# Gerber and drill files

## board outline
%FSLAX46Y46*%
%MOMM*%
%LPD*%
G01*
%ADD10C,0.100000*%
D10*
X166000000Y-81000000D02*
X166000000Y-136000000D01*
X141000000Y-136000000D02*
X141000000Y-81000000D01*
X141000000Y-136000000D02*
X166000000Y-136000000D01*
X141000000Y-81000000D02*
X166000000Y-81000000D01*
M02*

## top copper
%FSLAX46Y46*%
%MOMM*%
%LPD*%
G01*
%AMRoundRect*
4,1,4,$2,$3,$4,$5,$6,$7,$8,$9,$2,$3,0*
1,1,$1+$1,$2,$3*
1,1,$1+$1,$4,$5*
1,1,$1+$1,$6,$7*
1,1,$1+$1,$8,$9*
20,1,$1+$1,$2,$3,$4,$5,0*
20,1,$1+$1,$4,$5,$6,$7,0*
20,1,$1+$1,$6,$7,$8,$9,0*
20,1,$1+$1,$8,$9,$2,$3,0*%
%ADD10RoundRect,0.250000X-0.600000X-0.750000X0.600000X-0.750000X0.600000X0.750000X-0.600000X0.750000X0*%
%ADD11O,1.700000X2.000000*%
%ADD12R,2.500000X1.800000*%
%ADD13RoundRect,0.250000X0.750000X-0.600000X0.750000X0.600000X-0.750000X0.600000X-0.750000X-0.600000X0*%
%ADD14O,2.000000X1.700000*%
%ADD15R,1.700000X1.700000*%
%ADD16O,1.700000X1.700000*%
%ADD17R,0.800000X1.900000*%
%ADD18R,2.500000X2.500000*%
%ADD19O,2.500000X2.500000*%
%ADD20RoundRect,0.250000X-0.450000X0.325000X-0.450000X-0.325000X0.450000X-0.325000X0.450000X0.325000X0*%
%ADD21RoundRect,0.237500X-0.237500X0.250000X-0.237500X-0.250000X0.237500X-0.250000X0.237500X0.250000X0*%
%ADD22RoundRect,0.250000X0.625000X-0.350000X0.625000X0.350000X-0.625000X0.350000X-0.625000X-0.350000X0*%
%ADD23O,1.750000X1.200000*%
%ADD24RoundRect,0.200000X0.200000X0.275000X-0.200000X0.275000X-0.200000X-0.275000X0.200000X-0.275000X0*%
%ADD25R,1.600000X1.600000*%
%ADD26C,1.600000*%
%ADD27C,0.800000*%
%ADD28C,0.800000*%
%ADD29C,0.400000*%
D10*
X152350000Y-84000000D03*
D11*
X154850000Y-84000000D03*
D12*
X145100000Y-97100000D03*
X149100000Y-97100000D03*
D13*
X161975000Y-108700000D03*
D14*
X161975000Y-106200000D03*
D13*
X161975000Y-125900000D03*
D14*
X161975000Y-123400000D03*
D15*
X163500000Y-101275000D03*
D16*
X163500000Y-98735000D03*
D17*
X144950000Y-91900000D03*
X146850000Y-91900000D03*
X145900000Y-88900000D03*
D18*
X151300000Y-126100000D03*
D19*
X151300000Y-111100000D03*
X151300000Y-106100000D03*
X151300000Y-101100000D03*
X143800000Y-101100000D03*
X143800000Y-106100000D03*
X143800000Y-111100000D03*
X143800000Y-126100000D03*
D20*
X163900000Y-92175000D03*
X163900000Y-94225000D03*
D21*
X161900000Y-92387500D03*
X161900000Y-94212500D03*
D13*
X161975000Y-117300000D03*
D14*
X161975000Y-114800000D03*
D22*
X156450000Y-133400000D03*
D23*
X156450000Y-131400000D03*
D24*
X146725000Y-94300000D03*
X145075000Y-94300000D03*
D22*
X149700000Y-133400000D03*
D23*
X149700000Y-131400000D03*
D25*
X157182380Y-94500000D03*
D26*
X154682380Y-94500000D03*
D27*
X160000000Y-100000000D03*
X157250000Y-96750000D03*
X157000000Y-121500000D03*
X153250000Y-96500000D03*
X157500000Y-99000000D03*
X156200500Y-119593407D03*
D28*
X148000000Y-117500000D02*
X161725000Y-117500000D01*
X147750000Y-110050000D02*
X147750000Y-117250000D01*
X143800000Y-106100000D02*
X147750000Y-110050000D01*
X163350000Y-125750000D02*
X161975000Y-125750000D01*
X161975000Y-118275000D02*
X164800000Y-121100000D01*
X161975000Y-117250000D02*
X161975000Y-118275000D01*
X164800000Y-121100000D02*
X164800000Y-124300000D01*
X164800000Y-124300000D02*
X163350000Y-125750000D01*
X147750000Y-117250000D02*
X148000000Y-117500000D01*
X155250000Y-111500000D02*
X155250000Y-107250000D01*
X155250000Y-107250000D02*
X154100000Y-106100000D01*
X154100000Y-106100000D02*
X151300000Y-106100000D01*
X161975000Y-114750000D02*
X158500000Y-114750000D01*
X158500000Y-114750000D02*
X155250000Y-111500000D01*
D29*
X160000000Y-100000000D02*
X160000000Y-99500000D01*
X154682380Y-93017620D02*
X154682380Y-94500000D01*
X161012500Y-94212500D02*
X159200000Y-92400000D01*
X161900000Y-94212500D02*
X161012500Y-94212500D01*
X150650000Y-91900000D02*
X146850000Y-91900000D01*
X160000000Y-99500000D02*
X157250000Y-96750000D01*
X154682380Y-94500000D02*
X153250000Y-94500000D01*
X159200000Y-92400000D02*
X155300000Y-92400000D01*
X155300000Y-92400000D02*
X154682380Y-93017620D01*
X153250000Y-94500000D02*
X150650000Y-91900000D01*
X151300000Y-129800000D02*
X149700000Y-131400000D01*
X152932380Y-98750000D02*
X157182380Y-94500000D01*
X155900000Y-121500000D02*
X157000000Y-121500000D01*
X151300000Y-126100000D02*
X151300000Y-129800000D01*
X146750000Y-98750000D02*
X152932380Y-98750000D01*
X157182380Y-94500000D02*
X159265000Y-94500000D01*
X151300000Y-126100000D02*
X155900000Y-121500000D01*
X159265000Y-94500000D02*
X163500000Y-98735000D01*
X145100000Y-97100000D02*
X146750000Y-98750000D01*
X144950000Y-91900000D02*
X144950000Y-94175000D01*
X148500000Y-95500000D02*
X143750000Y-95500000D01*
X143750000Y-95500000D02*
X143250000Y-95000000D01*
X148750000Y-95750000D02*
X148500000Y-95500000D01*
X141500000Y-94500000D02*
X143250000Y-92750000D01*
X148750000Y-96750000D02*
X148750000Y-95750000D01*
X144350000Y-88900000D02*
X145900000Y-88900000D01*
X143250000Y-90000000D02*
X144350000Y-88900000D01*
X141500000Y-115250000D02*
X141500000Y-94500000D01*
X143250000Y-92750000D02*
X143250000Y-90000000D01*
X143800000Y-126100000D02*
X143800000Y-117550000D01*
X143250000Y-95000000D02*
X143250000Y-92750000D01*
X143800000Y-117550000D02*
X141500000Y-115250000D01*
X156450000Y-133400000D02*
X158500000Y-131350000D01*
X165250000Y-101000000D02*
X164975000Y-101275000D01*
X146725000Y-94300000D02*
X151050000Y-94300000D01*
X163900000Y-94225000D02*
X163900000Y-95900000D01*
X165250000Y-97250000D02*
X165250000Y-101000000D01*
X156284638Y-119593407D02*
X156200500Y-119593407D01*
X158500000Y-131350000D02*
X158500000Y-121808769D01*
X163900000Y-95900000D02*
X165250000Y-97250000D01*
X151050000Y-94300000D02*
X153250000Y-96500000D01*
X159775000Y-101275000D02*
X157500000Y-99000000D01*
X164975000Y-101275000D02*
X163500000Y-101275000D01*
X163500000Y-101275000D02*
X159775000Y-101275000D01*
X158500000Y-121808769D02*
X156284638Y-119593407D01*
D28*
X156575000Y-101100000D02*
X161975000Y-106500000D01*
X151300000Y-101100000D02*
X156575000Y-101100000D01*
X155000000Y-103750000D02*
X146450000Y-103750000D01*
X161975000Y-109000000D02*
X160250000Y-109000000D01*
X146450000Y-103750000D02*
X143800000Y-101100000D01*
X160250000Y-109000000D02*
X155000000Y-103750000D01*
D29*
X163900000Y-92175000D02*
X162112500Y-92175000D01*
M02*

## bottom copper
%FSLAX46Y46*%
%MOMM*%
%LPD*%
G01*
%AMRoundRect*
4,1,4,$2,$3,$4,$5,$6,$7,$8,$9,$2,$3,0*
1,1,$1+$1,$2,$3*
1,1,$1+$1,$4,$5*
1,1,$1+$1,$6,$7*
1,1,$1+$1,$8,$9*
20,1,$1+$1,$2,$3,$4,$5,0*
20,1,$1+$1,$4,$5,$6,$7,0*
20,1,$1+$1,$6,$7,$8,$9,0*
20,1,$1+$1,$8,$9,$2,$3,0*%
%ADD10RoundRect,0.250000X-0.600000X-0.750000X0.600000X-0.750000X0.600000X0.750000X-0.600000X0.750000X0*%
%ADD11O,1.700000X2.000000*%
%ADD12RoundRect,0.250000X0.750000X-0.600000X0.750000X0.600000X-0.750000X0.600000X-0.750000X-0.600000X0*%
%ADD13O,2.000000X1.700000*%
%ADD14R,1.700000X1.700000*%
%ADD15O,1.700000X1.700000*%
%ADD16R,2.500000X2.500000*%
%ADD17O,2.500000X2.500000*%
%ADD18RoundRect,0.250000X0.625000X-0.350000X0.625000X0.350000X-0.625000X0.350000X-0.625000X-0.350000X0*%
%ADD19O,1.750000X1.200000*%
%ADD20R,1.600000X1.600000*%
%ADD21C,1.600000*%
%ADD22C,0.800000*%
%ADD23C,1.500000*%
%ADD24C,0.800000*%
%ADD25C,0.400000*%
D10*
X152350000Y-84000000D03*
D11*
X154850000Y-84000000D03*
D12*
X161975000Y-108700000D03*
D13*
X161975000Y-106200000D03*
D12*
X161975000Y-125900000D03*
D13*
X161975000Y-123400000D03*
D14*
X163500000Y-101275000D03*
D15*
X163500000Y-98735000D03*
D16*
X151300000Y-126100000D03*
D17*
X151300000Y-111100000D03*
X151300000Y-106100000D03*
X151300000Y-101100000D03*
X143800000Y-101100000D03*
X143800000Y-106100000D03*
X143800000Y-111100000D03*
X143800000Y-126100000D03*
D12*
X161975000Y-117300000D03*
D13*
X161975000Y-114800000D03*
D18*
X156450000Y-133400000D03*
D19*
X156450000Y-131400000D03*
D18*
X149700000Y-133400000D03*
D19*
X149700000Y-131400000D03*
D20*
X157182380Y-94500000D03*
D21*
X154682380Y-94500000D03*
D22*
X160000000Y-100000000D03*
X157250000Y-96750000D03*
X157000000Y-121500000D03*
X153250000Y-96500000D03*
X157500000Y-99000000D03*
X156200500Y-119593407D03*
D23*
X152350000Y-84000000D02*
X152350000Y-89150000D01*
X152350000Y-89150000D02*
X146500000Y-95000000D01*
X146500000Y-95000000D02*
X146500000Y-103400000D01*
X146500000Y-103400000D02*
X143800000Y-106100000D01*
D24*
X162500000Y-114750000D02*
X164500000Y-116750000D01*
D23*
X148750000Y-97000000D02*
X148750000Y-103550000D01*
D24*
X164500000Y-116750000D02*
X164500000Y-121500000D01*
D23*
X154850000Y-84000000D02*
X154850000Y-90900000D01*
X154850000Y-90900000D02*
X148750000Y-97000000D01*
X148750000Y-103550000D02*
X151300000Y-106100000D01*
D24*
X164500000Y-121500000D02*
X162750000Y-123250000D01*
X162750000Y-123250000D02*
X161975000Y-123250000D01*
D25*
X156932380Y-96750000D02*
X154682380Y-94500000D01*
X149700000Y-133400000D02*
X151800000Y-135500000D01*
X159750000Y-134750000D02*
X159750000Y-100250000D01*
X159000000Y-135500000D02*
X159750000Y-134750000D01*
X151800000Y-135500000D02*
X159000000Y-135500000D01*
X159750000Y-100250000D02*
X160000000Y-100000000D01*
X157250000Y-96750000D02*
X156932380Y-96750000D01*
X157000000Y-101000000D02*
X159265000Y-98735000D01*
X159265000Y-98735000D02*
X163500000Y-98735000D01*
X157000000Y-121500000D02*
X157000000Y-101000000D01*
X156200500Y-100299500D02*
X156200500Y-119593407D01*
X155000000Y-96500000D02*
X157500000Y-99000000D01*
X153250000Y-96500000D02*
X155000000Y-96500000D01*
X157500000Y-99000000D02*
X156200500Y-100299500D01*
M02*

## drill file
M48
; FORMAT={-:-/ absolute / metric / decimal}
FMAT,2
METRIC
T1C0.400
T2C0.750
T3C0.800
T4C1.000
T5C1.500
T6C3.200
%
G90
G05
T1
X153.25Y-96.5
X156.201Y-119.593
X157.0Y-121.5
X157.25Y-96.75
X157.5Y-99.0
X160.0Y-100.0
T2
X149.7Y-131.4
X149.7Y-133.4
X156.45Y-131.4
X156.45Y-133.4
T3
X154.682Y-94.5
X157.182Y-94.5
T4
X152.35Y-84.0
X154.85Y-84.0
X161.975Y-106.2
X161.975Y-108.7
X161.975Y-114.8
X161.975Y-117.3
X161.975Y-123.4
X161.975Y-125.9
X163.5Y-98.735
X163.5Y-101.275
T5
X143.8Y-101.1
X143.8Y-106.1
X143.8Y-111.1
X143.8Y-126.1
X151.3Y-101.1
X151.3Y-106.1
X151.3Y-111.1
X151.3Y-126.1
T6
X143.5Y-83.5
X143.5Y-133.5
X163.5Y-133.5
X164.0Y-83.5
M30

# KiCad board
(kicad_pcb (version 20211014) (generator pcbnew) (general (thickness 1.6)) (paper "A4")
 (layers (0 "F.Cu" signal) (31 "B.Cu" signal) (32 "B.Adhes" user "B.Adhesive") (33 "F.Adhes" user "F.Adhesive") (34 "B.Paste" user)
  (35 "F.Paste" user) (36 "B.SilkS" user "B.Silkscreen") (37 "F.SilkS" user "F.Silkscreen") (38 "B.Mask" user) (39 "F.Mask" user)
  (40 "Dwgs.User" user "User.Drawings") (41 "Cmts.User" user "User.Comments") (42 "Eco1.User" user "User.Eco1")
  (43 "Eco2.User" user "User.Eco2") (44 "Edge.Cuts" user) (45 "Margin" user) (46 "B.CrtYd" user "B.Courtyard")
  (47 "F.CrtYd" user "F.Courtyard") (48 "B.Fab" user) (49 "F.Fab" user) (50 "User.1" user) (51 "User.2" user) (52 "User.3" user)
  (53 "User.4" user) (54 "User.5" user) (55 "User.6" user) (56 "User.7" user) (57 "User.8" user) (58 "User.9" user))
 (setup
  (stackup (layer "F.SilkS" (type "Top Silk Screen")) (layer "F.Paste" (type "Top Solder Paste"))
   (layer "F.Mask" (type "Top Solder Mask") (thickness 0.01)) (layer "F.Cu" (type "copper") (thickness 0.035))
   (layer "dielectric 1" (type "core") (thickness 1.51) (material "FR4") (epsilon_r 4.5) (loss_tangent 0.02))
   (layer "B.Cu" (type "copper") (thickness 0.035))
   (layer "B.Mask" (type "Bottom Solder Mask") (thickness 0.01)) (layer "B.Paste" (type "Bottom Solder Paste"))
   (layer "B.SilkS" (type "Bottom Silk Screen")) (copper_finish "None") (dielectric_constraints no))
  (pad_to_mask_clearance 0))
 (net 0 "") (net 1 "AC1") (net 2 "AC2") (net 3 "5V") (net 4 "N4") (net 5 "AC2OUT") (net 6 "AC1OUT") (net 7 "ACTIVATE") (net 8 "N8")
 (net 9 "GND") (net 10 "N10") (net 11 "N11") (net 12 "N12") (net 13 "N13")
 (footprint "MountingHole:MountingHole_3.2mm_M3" (layer "F.Cu") (at 163.5 133.5)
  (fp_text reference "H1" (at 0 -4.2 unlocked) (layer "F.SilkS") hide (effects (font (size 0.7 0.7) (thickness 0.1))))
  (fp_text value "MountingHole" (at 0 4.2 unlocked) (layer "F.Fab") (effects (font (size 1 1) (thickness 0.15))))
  (pad "" np_thru_hole circle (at 0 0) (size 3.2 3.2) (drill 3.2) (layers *.Cu *.Mask)))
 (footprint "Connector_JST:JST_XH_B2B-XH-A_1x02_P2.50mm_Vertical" (layer "F.Cu") (at 152.35 84)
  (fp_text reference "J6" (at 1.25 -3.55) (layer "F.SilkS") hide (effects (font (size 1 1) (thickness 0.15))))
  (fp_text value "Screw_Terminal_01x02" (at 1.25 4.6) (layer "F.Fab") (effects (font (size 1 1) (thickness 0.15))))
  (pad "1" thru_hole roundrect (at 0 0) (size 1.7 2) (drill 1) (layers *.Cu *.Mask) (roundrect_rratio 0.1470588235) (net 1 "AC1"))
  (pad "2" thru_hole oval (at 2.5 0) (size 1.7 2) (drill 1) (layers *.Cu *.Mask) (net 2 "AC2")))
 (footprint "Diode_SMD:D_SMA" (layer "F.Cu") (at 147.1 97.1)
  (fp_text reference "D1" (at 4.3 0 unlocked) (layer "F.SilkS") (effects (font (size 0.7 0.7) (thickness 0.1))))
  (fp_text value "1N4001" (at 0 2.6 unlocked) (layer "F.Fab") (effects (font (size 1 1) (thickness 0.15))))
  (pad "1" smd rect (at -2 0) (size 2.5 1.8) (layers "F.Cu" "F.Paste" "F.Mask") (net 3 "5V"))
  (pad "2" smd rect (at 2 0) (size 2.5 1.8) (layers "F.Cu" "F.Paste" "F.Mask") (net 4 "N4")))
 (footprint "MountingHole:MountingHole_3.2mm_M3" (layer "F.Cu") (at 164 83.5)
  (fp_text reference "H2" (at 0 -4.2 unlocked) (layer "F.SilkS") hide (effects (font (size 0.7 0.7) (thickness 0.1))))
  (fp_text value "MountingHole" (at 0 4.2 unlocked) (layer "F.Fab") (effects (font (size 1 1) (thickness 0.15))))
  (pad "" np_thru_hole circle (at 0 0) (size 3.2 3.2) (drill 3.2) (layers *.Cu *.Mask)))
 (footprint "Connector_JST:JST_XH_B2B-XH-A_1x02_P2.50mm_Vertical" (layer "F.Cu") (at 161.975 108.7 90)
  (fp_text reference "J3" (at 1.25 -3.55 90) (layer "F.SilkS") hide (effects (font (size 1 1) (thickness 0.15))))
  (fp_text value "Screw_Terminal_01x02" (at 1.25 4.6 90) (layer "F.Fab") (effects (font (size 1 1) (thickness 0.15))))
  (pad "1" thru_hole roundrect (at 0 0 90) (size 1.7 2) (drill 1) (layers *.Cu *.Mask) (roundrect_rratio 0.1470588235) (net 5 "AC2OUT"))
  (pad "2" thru_hole oval (at 2.5 0 90) (size 1.7 2) (drill 1) (layers *.Cu *.Mask) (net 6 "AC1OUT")))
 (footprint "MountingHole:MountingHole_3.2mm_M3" (layer "F.Cu") (at 143.5 83.5)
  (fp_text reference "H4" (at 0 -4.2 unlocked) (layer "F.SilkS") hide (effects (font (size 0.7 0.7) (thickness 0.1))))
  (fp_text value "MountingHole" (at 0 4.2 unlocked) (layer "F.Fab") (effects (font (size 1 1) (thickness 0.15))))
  (pad "" np_thru_hole circle (at 0 0) (size 3.2 3.2) (drill 3.2) (layers *.Cu *.Mask)))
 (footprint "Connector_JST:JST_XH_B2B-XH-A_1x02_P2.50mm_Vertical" (layer "F.Cu") (at 161.975 125.9 90)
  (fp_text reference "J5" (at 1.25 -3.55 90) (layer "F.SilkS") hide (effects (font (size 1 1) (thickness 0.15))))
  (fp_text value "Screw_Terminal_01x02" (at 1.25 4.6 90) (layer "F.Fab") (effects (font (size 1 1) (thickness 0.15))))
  (pad "1" thru_hole roundrect (at 0 0 90) (size 1.7 2) (drill 1) (layers *.Cu *.Mask) (roundrect_rratio 0.1470588235) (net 1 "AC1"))
  (pad "2" thru_hole oval (at 2.5 0 90) (size 1.7 2) (drill 1) (layers *.Cu *.Mask) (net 2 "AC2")))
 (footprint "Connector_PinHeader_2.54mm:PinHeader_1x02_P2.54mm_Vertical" (layer "F.Cu") (at 163.5 101.275 180)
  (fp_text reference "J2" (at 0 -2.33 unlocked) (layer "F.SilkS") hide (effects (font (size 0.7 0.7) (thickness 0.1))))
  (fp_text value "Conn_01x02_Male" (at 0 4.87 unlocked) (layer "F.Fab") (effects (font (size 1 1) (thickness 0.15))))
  (pad "1" thru_hole rect (at 0 0 180) (size 1.7 1.7) (drill 1) (layers *.Cu *.Mask) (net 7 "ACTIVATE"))
  (pad "2" thru_hole oval (at 0 2.54 180) (size 1.7 1.7) (drill 1) (layers *.Cu *.Mask) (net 3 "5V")))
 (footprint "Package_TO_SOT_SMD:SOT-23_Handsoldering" (layer "F.Cu") (at 145.9 90.4 90)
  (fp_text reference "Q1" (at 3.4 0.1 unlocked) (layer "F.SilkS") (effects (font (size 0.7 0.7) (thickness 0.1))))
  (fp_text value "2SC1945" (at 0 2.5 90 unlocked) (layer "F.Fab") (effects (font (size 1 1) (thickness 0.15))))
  (pad "1" smd rect (at -1.5 -0.95 90) (size 1.9 0.8) (layers "F.Cu" "F.Paste" "F.Mask") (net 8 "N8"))
  (pad "2" smd rect (at -1.5 0.95 90) (size 1.9 0.8) (layers "F.Cu" "F.Paste" "F.Mask") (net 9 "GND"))
  (pad "3" smd rect (at 1.5 0 90) (size 1.9 0.8) (layers "F.Cu" "F.Paste" "F.Mask") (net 4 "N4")))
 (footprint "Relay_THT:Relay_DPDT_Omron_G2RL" (layer "F.Cu") (at 151.3 126.1 90)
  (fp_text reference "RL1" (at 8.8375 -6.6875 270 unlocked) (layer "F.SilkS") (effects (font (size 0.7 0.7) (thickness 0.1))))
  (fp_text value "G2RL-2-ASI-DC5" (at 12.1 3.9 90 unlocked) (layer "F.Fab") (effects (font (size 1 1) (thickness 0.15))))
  (pad "1" thru_hole rect (at 0 0 180) (size 2.5 2.5) (drill 1.5) (layers *.Cu *.Mask) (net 3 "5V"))
  (pad "2" thru_hole oval (at 15 0 180) (size 2.5 2.5) (drill 1.5) (layers *.Cu *.Mask) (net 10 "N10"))
  (pad "3" thru_hole oval (at 20 0 180) (size 2.5 2.5) (drill 1.5) (layers *.Cu *.Mask) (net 2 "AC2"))
  (pad "4" thru_hole oval (at 25 0 180) (size 2.5 2.5) (drill 1.5) (layers *.Cu *.Mask) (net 6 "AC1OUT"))
  (pad "5" thru_hole oval (at 25 -7.5 180) (size 2.5 2.5) (drill 1.5) (layers *.Cu *.Mask) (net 5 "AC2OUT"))
  (pad "6" thru_hole oval (at 20 -7.5 180) (size 2.5 2.5) (drill 1.5) (layers *.Cu *.Mask) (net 1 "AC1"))
  (pad "7" thru_hole oval (at 15 -7.5 180) (size 2.5 2.5) (drill 1.5) (layers *.Cu *.Mask) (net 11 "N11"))
  (pad "8" thru_hole oval (at 0 -7.5 180) (size 2.5 2.5) (drill 1.5) (layers *.Cu *.Mask) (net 4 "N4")))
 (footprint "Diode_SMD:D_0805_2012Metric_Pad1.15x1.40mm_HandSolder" (layer "F.Cu") (at 163.9 93.2 -90)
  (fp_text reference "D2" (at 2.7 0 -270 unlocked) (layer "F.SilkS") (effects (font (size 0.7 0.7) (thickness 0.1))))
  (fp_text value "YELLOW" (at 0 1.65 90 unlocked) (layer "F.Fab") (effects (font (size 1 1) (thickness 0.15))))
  (pad "1" smd roundrect (at -1.025 0 270) (size 1.15 1.4) (layers "F.Cu" "F.Paste" "F.Mask") (roundrect_rratio 0.2173913043) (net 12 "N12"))
  (pad "2" smd roundrect (at 1.025 0 270) (size 1.15 1.4) (layers "F.Cu" "F.Paste" "F.Mask") (roundrect_rratio 0.2173913043)
   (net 7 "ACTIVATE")))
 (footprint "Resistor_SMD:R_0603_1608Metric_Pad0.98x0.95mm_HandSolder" (layer "F.Cu") (at 161.9 93.3 -90)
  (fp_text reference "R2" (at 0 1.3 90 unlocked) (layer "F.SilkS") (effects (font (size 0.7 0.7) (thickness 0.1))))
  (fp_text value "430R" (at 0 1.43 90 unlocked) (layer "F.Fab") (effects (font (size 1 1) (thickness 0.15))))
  (pad "1" smd roundrect (at -0.9125 0 270) (size 0.975 0.95) (layers "F.Cu" "F.Paste" "F.Mask") (roundrect_rratio 0.25) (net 12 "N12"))
  (pad "2" smd roundrect (at 0.9125 0 270) (size 0.975 0.95) (layers "F.Cu" "F.Paste" "F.Mask") (roundrect_rratio 0.25) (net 9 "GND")))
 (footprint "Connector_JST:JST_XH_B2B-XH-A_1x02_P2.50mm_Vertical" (layer "F.Cu") (at 161.975 117.3 90)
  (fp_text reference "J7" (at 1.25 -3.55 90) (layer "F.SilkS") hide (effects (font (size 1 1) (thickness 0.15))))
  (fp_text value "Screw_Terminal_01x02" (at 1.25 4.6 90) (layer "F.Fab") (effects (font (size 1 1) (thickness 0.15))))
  (pad "1" thru_hole roundrect (at 0 0 90) (size 1.7 2) (drill 1) (layers *.Cu *.Mask) (roundrect_rratio 0.1470588235) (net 1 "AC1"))
  (pad "2" thru_hole oval (at 2.5 0 90) (size 1.7 2) (drill 1) (layers *.Cu *.Mask) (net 2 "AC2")))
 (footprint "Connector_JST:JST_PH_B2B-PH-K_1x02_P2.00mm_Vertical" (layer "F.Cu") (at 156.45 133.4 90)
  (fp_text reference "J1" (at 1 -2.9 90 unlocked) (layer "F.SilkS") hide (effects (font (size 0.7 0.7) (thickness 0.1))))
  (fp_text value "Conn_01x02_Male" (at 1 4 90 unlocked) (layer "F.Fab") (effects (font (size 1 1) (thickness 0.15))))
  (pad "1" thru_hole roundrect (at 0 0 90) (size 1.2 1.75) (drill 0.75) (layers *.Cu *.Mask) (roundrect_rratio 0.2083333333)
   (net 7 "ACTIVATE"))
  (pad "2" thru_hole oval (at 2 0 90) (size 1.2 1.75) (drill 0.75) (layers *.Cu *.Mask) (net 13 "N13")))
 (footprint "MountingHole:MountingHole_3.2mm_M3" (layer "F.Cu") (at 143.5 133.5)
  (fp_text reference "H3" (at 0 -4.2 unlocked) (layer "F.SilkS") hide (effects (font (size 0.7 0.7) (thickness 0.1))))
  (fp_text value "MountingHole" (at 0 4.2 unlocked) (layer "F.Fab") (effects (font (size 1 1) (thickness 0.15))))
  (pad "" np_thru_hole circle (at 0 0) (size 3.2 3.2) (drill 3.2) (layers *.Cu *.Mask)))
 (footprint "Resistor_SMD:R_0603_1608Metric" (layer "F.Cu") (at 145.9 94.3 180)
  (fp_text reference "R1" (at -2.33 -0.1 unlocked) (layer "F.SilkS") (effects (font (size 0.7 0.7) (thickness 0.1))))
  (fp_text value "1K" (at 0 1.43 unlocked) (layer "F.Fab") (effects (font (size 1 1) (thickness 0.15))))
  (pad "1" smd roundrect (at -0.825 0 180) (size 0.8 0.95) (layers "F.Cu" "F.Paste" "F.Mask") (roundrect_rratio 0.25) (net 7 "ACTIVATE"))
  (pad "2" smd roundrect (at 0.825 0 180) (size 0.8 0.95) (layers "F.Cu" "F.Paste" "F.Mask") (roundrect_rratio 0.25) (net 8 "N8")))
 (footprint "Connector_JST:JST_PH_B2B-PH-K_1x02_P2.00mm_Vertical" (layer "F.Cu") (at 149.7 133.4 90)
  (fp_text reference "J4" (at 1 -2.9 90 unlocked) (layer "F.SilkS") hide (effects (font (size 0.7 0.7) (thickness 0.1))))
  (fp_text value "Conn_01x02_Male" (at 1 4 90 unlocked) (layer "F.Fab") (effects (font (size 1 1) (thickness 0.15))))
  (pad "1" thru_hole roundrect (at 0 0 90) (size 1.2 1.75) (drill 0.75) (layers *.Cu *.Mask) (roundrect_rratio 0.2083333333) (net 9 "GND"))
  (pad "2" thru_hole oval (at 2 0 90) (size 1.2 1.75) (drill 0.75) (layers *.Cu *.Mask) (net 3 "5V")))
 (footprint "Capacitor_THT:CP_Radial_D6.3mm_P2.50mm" (layer "F.Cu") (at 157.18238 94.5 180)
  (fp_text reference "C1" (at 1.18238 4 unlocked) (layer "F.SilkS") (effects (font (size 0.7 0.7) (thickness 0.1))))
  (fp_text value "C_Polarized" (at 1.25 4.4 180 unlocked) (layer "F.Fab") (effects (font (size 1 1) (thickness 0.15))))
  (pad "1" thru_hole rect (at 0 0 180) (size 1.6 1.6) (drill 0.8) (layers *.Cu *.Mask) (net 3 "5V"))
  (pad "2" thru_hole circle (at 2.5 0 180) (size 1.6 1.6) (drill 0.8) (layers *.Cu *.Mask) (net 9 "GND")))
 (gr_line (start 166 81) (end 166 136) (layer "Edge.Cuts") (width 0.1))
 (gr_line (start 141 136) (end 141 81) (layer "Edge.Cuts") (width 0.1))
 (gr_line (start 141 136) (end 166 136) (layer "Edge.Cuts") (width 0.1))
 (gr_line (start 141 81) (end 166 81) (layer "Edge.Cuts") (width 0.1))
 (segment (start 148 117.5) (end 161.725 117.5) (width 0.8) (layer "F.Cu") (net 1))
 (segment (start 147.75 110.05) (end 147.75 117.25) (width 0.8) (layer "F.Cu") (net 1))
 (segment (start 143.8 106.1) (end 147.75 110.05) (width 0.8) (layer "F.Cu") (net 1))
 (segment (start 163.35 125.75) (end 161.975 125.75) (width 0.8) (layer "F.Cu") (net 1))
 (segment (start 161.975 118.275) (end 164.8 121.1) (width 0.8) (layer "F.Cu") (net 1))
 (segment (start 161.975 117.25) (end 161.975 118.275) (width 0.8) (layer "F.Cu") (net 1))
 (segment (start 164.8 121.1) (end 164.8 124.3) (width 0.8) (layer "F.Cu") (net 1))
 (segment (start 164.8 124.3) (end 163.35 125.75) (width 0.8) (layer "F.Cu") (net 1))
 (segment (start 147.75 117.25) (end 148 117.5) (width 0.8) (layer "F.Cu") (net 1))
 (segment (start 152.35 84) (end 152.35 89.15) (width 1.5) (layer "B.Cu") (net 1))
 (segment (start 152.35 89.15) (end 146.5 95) (width 1.5) (layer "B.Cu") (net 1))
 (segment (start 146.5 95) (end 146.5 103.4) (width 1.5) (layer "B.Cu") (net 1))
 (segment (start 146.5 103.4) (end 143.8 106.1) (width 1.5) (layer "B.Cu") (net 1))
 (segment (start 155.25 111.5) (end 155.25 107.25) (width 0.8) (layer "F.Cu") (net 2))
 (segment (start 155.25 107.25) (end 154.1 106.1) (width 0.8) (layer "F.Cu") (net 2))
 (segment (start 154.1 106.1) (end 151.3 106.1) (width 0.8) (layer "F.Cu") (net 2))
 (segment (start 161.975 114.75) (end 158.5 114.75) (width 0.8) (layer "F.Cu") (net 2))
 (segment (start 158.5 114.75) (end 155.25 111.5) (width 0.8) (layer "F.Cu") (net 2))
 (segment (start 162.5 114.75) (end 164.5 116.75) (width 0.8) (layer "B.Cu") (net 2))
 (segment (start 148.75 97) (end 148.75 103.55) (width 1.5) (layer "B.Cu") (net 2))
 (segment (start 164.5 116.75) (end 164.5 121.5) (width 0.8) (layer "B.Cu") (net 2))
 (segment (start 154.85 84) (end 154.85 90.9) (width 1.5) (layer "B.Cu") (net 2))
 (segment (start 154.85 90.9) (end 148.75 97) (width 1.5) (layer "B.Cu") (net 2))
 (segment (start 148.75 103.55) (end 151.3 106.1) (width 1.5) (layer "B.Cu") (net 2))
 (segment (start 164.5 121.5) (end 162.75 123.25) (width 0.8) (layer "B.Cu") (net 2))
 (segment (start 162.75 123.25) (end 161.975 123.25) (width 0.8) (layer "B.Cu") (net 2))
 (segment (start 160 100) (end 160 99.5) (width 0.4) (layer "F.Cu") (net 9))
 (segment (start 154.68238 93.01762) (end 154.68238 94.5) (width 0.4) (layer "F.Cu") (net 9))
 (segment (start 161.0125 94.2125) (end 159.2 92.4) (width 0.4) (layer "F.Cu") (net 9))
 (segment (start 161.9 94.2125) (end 161.0125 94.2125) (width 0.4) (layer "F.Cu") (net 9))
 (segment (start 150.65 91.9) (end 146.85 91.9) (width 0.4) (layer "F.Cu") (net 9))
 (segment (start 160 99.5) (end 157.25 96.75) (width 0.4) (layer "F.Cu") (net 9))
 (segment (start 154.68238 94.5) (end 153.25 94.5) (width 0.4) (layer "F.Cu") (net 9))
 (segment (start 159.2 92.4) (end 155.3 92.4) (width 0.4) (layer "F.Cu") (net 9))
 (segment (start 155.3 92.4) (end 154.68238 93.01762) (width 0.4) (layer "F.Cu") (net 9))
 (segment (start 153.25 94.5) (end 150.65 91.9) (width 0.4) (layer "F.Cu") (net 9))
 (via (at 160 100) (size 0.8) (drill 0.4) (layers "F.Cu" "B.Cu") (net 9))
 (via (at 157.25 96.75) (size 0.8) (drill 0.4) (layers "F.Cu" "B.Cu") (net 9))
 (segment (start 156.93238 96.75) (end 154.68238 94.5) (width 0.4) (layer "B.Cu") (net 9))
 (segment (start 149.7 133.4) (end 151.8 135.5) (width 0.4) (layer "B.Cu") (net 9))
 (segment (start 159.75 134.75) (end 159.75 100.25) (width 0.4) (layer "B.Cu") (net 9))
 (segment (start 159 135.5) (end 159.75 134.75) (width 0.4) (layer "B.Cu") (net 9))
 (segment (start 151.8 135.5) (end 159 135.5) (width 0.4) (layer "B.Cu") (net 9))
 (segment (start 159.75 100.25) (end 160 100) (width 0.4) (layer "B.Cu") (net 9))
 (segment (start 157.25 96.75) (end 156.93238 96.75) (width 0.4) (layer "B.Cu") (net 9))
 (segment (start 151.3 129.8) (end 149.7 131.4) (width 0.4) (layer "F.Cu") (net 3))
 (segment (start 152.93238 98.75) (end 157.18238 94.5) (width 0.4) (layer "F.Cu") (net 3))
 (segment (start 155.9 121.5) (end 157 121.5) (width 0.4) (layer "F.Cu") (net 3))
 (segment (start 151.3 126.1) (end 151.3 129.8) (width 0.4) (layer "F.Cu") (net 3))
 (segment (start 146.75 98.75) (end 152.93238 98.75) (width 0.4) (layer "F.Cu") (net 3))
 (segment (start 157.18238 94.5) (end 159.265 94.5) (width 0.4) (layer "F.Cu") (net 3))
 (segment (start 151.3 126.1) (end 155.9 121.5) (width 0.4) (layer "F.Cu") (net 3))
 (segment (start 159.265 94.5) (end 163.5 98.735) (width 0.4) (layer "F.Cu") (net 3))
 (segment (start 145.1 97.1) (end 146.75 98.75) (width 0.4) (layer "F.Cu") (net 3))
 (via (at 157 121.5) (size 0.8) (drill 0.4) (layers "F.Cu" "B.Cu") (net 3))
 (segment (start 157 101) (end 159.265 98.735) (width 0.4) (layer "B.Cu") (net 3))
 (segment (start 159.265 98.735) (end 163.5 98.735) (width 0.4) (layer "B.Cu") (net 3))
 (segment (start 157 121.5) (end 157 101) (width 0.4) (layer "B.Cu") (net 3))
 (segment (start 144.95 91.9) (end 144.95 94.175) (width 0.4) (layer "F.Cu") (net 8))
 (segment (start 148.5 95.5) (end 143.75 95.5) (width 0.4) (layer "F.Cu") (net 4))
 (segment (start 143.75 95.5) (end 143.25 95) (width 0.4) (layer "F.Cu") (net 4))
 (segment (start 148.75 95.75) (end 148.5 95.5) (width 0.4) (layer "F.Cu") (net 4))
 (segment (start 141.5 94.5) (end 143.25 92.75) (width 0.4) (layer "F.Cu") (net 4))
 (segment (start 148.75 96.75) (end 148.75 95.75) (width 0.4) (layer "F.Cu") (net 4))
 (segment (start 144.35 88.9) (end 145.9 88.9) (width 0.4) (layer "F.Cu") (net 4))
 (segment (start 143.25 90) (end 144.35 88.9) (width 0.4) (layer "F.Cu") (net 4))
 (segment (start 141.5 115.25) (end 141.5 94.5) (width 0.4) (layer "F.Cu") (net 4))
 (segment (start 143.25 92.75) (end 143.25 90) (width 0.4) (layer "F.Cu") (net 4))
 (segment (start 143.8 126.1) (end 143.8 117.55) (width 0.4) (layer "F.Cu") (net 4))
 (segment (start 143.25 95) (end 143.25 92.75) (width 0.4) (layer "F.Cu") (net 4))
 (segment (start 143.8 117.55) (end 141.5 115.25) (width 0.4) (layer "F.Cu") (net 4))
 (segment (start 156.45 133.4) (end 158.5 131.35) (width 0.4) (layer "F.Cu") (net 7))
 (segment (start 165.25 101) (end 164.975 101.275) (width 0.4) (layer "F.Cu") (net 7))
 (segment (start 146.725 94.3) (end 151.05 94.3) (width 0.4) (layer "F.Cu") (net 7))
 (segment (start 163.9 94.225) (end 163.9 95.9) (width 0.4) (layer "F.Cu") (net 7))
 (segment (start 165.25 97.25) (end 165.25 101) (width 0.4) (layer "F.Cu") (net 7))
 (segment (start 156.284638 119.593407) (end 156.2005 119.593407) (width 0.4) (layer "F.Cu") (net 7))
 (segment (start 158.5 131.35) (end 158.5 121.808769) (width 0.4) (layer "F.Cu") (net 7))
 (segment (start 163.9 95.9) (end 165.25 97.25) (width 0.4) (layer "F.Cu") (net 7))
 (segment (start 151.05 94.3) (end 153.25 96.5) (width 0.4) (layer "F.Cu") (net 7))
 (segment (start 159.775 101.275) (end 157.5 99) (width 0.4) (layer "F.Cu") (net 7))
 (segment (start 164.975 101.275) (end 163.5 101.275) (width 0.4) (layer "F.Cu") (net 7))
 (segment (start 163.5 101.275) (end 159.775 101.275) (width 0.4) (layer "F.Cu") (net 7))
 (segment (start 158.5 121.808769) (end 156.284638 119.593407) (width 0.4) (layer "F.Cu") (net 7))
 (via (at 153.25 96.5) (size 0.8) (drill 0.4) (layers "F.Cu" "B.Cu") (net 7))
 (via (at 157.5 99) (size 0.8) (drill 0.4) (layers "F.Cu" "B.Cu") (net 7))
 (via (at 156.2005 119.593407) (size 0.8) (drill 0.4) (layers "F.Cu" "B.Cu") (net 7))
 (segment (start 156.2005 100.2995) (end 156.2005 119.593407) (width 0.4) (layer "B.Cu") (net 7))
 (segment (start 155 96.5) (end 157.5 99) (width 0.4) (layer "B.Cu") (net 7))
 (segment (start 153.25 96.5) (end 155 96.5) (width 0.4) (layer "B.Cu") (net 7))
 (segment (start 157.5 99) (end 156.2005 100.2995) (width 0.4) (layer "B.Cu") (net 7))
 (segment (start 156.575 101.1) (end 161.975 106.5) (width 0.8) (layer "F.Cu") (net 6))
 (segment (start 151.3 101.1) (end 156.575 101.1) (width 0.8) (layer "F.Cu") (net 6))
 (segment (start 155 103.75) (end 146.45 103.75) (width 0.8) (layer "F.Cu") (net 5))
 (segment (start 161.975 109) (end 160.25 109) (width 0.8) (layer "F.Cu") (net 5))
 (segment (start 146.45 103.75) (end 143.8 101.1) (width 0.8) (layer "F.Cu") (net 5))
 (segment (start 160.25 109) (end 155 103.75) (width 0.8) (layer "F.Cu") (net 5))
 (segment (start 163.9 92.175) (end 162.1125 92.175) (width 0.4) (layer "F.Cu") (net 12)))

